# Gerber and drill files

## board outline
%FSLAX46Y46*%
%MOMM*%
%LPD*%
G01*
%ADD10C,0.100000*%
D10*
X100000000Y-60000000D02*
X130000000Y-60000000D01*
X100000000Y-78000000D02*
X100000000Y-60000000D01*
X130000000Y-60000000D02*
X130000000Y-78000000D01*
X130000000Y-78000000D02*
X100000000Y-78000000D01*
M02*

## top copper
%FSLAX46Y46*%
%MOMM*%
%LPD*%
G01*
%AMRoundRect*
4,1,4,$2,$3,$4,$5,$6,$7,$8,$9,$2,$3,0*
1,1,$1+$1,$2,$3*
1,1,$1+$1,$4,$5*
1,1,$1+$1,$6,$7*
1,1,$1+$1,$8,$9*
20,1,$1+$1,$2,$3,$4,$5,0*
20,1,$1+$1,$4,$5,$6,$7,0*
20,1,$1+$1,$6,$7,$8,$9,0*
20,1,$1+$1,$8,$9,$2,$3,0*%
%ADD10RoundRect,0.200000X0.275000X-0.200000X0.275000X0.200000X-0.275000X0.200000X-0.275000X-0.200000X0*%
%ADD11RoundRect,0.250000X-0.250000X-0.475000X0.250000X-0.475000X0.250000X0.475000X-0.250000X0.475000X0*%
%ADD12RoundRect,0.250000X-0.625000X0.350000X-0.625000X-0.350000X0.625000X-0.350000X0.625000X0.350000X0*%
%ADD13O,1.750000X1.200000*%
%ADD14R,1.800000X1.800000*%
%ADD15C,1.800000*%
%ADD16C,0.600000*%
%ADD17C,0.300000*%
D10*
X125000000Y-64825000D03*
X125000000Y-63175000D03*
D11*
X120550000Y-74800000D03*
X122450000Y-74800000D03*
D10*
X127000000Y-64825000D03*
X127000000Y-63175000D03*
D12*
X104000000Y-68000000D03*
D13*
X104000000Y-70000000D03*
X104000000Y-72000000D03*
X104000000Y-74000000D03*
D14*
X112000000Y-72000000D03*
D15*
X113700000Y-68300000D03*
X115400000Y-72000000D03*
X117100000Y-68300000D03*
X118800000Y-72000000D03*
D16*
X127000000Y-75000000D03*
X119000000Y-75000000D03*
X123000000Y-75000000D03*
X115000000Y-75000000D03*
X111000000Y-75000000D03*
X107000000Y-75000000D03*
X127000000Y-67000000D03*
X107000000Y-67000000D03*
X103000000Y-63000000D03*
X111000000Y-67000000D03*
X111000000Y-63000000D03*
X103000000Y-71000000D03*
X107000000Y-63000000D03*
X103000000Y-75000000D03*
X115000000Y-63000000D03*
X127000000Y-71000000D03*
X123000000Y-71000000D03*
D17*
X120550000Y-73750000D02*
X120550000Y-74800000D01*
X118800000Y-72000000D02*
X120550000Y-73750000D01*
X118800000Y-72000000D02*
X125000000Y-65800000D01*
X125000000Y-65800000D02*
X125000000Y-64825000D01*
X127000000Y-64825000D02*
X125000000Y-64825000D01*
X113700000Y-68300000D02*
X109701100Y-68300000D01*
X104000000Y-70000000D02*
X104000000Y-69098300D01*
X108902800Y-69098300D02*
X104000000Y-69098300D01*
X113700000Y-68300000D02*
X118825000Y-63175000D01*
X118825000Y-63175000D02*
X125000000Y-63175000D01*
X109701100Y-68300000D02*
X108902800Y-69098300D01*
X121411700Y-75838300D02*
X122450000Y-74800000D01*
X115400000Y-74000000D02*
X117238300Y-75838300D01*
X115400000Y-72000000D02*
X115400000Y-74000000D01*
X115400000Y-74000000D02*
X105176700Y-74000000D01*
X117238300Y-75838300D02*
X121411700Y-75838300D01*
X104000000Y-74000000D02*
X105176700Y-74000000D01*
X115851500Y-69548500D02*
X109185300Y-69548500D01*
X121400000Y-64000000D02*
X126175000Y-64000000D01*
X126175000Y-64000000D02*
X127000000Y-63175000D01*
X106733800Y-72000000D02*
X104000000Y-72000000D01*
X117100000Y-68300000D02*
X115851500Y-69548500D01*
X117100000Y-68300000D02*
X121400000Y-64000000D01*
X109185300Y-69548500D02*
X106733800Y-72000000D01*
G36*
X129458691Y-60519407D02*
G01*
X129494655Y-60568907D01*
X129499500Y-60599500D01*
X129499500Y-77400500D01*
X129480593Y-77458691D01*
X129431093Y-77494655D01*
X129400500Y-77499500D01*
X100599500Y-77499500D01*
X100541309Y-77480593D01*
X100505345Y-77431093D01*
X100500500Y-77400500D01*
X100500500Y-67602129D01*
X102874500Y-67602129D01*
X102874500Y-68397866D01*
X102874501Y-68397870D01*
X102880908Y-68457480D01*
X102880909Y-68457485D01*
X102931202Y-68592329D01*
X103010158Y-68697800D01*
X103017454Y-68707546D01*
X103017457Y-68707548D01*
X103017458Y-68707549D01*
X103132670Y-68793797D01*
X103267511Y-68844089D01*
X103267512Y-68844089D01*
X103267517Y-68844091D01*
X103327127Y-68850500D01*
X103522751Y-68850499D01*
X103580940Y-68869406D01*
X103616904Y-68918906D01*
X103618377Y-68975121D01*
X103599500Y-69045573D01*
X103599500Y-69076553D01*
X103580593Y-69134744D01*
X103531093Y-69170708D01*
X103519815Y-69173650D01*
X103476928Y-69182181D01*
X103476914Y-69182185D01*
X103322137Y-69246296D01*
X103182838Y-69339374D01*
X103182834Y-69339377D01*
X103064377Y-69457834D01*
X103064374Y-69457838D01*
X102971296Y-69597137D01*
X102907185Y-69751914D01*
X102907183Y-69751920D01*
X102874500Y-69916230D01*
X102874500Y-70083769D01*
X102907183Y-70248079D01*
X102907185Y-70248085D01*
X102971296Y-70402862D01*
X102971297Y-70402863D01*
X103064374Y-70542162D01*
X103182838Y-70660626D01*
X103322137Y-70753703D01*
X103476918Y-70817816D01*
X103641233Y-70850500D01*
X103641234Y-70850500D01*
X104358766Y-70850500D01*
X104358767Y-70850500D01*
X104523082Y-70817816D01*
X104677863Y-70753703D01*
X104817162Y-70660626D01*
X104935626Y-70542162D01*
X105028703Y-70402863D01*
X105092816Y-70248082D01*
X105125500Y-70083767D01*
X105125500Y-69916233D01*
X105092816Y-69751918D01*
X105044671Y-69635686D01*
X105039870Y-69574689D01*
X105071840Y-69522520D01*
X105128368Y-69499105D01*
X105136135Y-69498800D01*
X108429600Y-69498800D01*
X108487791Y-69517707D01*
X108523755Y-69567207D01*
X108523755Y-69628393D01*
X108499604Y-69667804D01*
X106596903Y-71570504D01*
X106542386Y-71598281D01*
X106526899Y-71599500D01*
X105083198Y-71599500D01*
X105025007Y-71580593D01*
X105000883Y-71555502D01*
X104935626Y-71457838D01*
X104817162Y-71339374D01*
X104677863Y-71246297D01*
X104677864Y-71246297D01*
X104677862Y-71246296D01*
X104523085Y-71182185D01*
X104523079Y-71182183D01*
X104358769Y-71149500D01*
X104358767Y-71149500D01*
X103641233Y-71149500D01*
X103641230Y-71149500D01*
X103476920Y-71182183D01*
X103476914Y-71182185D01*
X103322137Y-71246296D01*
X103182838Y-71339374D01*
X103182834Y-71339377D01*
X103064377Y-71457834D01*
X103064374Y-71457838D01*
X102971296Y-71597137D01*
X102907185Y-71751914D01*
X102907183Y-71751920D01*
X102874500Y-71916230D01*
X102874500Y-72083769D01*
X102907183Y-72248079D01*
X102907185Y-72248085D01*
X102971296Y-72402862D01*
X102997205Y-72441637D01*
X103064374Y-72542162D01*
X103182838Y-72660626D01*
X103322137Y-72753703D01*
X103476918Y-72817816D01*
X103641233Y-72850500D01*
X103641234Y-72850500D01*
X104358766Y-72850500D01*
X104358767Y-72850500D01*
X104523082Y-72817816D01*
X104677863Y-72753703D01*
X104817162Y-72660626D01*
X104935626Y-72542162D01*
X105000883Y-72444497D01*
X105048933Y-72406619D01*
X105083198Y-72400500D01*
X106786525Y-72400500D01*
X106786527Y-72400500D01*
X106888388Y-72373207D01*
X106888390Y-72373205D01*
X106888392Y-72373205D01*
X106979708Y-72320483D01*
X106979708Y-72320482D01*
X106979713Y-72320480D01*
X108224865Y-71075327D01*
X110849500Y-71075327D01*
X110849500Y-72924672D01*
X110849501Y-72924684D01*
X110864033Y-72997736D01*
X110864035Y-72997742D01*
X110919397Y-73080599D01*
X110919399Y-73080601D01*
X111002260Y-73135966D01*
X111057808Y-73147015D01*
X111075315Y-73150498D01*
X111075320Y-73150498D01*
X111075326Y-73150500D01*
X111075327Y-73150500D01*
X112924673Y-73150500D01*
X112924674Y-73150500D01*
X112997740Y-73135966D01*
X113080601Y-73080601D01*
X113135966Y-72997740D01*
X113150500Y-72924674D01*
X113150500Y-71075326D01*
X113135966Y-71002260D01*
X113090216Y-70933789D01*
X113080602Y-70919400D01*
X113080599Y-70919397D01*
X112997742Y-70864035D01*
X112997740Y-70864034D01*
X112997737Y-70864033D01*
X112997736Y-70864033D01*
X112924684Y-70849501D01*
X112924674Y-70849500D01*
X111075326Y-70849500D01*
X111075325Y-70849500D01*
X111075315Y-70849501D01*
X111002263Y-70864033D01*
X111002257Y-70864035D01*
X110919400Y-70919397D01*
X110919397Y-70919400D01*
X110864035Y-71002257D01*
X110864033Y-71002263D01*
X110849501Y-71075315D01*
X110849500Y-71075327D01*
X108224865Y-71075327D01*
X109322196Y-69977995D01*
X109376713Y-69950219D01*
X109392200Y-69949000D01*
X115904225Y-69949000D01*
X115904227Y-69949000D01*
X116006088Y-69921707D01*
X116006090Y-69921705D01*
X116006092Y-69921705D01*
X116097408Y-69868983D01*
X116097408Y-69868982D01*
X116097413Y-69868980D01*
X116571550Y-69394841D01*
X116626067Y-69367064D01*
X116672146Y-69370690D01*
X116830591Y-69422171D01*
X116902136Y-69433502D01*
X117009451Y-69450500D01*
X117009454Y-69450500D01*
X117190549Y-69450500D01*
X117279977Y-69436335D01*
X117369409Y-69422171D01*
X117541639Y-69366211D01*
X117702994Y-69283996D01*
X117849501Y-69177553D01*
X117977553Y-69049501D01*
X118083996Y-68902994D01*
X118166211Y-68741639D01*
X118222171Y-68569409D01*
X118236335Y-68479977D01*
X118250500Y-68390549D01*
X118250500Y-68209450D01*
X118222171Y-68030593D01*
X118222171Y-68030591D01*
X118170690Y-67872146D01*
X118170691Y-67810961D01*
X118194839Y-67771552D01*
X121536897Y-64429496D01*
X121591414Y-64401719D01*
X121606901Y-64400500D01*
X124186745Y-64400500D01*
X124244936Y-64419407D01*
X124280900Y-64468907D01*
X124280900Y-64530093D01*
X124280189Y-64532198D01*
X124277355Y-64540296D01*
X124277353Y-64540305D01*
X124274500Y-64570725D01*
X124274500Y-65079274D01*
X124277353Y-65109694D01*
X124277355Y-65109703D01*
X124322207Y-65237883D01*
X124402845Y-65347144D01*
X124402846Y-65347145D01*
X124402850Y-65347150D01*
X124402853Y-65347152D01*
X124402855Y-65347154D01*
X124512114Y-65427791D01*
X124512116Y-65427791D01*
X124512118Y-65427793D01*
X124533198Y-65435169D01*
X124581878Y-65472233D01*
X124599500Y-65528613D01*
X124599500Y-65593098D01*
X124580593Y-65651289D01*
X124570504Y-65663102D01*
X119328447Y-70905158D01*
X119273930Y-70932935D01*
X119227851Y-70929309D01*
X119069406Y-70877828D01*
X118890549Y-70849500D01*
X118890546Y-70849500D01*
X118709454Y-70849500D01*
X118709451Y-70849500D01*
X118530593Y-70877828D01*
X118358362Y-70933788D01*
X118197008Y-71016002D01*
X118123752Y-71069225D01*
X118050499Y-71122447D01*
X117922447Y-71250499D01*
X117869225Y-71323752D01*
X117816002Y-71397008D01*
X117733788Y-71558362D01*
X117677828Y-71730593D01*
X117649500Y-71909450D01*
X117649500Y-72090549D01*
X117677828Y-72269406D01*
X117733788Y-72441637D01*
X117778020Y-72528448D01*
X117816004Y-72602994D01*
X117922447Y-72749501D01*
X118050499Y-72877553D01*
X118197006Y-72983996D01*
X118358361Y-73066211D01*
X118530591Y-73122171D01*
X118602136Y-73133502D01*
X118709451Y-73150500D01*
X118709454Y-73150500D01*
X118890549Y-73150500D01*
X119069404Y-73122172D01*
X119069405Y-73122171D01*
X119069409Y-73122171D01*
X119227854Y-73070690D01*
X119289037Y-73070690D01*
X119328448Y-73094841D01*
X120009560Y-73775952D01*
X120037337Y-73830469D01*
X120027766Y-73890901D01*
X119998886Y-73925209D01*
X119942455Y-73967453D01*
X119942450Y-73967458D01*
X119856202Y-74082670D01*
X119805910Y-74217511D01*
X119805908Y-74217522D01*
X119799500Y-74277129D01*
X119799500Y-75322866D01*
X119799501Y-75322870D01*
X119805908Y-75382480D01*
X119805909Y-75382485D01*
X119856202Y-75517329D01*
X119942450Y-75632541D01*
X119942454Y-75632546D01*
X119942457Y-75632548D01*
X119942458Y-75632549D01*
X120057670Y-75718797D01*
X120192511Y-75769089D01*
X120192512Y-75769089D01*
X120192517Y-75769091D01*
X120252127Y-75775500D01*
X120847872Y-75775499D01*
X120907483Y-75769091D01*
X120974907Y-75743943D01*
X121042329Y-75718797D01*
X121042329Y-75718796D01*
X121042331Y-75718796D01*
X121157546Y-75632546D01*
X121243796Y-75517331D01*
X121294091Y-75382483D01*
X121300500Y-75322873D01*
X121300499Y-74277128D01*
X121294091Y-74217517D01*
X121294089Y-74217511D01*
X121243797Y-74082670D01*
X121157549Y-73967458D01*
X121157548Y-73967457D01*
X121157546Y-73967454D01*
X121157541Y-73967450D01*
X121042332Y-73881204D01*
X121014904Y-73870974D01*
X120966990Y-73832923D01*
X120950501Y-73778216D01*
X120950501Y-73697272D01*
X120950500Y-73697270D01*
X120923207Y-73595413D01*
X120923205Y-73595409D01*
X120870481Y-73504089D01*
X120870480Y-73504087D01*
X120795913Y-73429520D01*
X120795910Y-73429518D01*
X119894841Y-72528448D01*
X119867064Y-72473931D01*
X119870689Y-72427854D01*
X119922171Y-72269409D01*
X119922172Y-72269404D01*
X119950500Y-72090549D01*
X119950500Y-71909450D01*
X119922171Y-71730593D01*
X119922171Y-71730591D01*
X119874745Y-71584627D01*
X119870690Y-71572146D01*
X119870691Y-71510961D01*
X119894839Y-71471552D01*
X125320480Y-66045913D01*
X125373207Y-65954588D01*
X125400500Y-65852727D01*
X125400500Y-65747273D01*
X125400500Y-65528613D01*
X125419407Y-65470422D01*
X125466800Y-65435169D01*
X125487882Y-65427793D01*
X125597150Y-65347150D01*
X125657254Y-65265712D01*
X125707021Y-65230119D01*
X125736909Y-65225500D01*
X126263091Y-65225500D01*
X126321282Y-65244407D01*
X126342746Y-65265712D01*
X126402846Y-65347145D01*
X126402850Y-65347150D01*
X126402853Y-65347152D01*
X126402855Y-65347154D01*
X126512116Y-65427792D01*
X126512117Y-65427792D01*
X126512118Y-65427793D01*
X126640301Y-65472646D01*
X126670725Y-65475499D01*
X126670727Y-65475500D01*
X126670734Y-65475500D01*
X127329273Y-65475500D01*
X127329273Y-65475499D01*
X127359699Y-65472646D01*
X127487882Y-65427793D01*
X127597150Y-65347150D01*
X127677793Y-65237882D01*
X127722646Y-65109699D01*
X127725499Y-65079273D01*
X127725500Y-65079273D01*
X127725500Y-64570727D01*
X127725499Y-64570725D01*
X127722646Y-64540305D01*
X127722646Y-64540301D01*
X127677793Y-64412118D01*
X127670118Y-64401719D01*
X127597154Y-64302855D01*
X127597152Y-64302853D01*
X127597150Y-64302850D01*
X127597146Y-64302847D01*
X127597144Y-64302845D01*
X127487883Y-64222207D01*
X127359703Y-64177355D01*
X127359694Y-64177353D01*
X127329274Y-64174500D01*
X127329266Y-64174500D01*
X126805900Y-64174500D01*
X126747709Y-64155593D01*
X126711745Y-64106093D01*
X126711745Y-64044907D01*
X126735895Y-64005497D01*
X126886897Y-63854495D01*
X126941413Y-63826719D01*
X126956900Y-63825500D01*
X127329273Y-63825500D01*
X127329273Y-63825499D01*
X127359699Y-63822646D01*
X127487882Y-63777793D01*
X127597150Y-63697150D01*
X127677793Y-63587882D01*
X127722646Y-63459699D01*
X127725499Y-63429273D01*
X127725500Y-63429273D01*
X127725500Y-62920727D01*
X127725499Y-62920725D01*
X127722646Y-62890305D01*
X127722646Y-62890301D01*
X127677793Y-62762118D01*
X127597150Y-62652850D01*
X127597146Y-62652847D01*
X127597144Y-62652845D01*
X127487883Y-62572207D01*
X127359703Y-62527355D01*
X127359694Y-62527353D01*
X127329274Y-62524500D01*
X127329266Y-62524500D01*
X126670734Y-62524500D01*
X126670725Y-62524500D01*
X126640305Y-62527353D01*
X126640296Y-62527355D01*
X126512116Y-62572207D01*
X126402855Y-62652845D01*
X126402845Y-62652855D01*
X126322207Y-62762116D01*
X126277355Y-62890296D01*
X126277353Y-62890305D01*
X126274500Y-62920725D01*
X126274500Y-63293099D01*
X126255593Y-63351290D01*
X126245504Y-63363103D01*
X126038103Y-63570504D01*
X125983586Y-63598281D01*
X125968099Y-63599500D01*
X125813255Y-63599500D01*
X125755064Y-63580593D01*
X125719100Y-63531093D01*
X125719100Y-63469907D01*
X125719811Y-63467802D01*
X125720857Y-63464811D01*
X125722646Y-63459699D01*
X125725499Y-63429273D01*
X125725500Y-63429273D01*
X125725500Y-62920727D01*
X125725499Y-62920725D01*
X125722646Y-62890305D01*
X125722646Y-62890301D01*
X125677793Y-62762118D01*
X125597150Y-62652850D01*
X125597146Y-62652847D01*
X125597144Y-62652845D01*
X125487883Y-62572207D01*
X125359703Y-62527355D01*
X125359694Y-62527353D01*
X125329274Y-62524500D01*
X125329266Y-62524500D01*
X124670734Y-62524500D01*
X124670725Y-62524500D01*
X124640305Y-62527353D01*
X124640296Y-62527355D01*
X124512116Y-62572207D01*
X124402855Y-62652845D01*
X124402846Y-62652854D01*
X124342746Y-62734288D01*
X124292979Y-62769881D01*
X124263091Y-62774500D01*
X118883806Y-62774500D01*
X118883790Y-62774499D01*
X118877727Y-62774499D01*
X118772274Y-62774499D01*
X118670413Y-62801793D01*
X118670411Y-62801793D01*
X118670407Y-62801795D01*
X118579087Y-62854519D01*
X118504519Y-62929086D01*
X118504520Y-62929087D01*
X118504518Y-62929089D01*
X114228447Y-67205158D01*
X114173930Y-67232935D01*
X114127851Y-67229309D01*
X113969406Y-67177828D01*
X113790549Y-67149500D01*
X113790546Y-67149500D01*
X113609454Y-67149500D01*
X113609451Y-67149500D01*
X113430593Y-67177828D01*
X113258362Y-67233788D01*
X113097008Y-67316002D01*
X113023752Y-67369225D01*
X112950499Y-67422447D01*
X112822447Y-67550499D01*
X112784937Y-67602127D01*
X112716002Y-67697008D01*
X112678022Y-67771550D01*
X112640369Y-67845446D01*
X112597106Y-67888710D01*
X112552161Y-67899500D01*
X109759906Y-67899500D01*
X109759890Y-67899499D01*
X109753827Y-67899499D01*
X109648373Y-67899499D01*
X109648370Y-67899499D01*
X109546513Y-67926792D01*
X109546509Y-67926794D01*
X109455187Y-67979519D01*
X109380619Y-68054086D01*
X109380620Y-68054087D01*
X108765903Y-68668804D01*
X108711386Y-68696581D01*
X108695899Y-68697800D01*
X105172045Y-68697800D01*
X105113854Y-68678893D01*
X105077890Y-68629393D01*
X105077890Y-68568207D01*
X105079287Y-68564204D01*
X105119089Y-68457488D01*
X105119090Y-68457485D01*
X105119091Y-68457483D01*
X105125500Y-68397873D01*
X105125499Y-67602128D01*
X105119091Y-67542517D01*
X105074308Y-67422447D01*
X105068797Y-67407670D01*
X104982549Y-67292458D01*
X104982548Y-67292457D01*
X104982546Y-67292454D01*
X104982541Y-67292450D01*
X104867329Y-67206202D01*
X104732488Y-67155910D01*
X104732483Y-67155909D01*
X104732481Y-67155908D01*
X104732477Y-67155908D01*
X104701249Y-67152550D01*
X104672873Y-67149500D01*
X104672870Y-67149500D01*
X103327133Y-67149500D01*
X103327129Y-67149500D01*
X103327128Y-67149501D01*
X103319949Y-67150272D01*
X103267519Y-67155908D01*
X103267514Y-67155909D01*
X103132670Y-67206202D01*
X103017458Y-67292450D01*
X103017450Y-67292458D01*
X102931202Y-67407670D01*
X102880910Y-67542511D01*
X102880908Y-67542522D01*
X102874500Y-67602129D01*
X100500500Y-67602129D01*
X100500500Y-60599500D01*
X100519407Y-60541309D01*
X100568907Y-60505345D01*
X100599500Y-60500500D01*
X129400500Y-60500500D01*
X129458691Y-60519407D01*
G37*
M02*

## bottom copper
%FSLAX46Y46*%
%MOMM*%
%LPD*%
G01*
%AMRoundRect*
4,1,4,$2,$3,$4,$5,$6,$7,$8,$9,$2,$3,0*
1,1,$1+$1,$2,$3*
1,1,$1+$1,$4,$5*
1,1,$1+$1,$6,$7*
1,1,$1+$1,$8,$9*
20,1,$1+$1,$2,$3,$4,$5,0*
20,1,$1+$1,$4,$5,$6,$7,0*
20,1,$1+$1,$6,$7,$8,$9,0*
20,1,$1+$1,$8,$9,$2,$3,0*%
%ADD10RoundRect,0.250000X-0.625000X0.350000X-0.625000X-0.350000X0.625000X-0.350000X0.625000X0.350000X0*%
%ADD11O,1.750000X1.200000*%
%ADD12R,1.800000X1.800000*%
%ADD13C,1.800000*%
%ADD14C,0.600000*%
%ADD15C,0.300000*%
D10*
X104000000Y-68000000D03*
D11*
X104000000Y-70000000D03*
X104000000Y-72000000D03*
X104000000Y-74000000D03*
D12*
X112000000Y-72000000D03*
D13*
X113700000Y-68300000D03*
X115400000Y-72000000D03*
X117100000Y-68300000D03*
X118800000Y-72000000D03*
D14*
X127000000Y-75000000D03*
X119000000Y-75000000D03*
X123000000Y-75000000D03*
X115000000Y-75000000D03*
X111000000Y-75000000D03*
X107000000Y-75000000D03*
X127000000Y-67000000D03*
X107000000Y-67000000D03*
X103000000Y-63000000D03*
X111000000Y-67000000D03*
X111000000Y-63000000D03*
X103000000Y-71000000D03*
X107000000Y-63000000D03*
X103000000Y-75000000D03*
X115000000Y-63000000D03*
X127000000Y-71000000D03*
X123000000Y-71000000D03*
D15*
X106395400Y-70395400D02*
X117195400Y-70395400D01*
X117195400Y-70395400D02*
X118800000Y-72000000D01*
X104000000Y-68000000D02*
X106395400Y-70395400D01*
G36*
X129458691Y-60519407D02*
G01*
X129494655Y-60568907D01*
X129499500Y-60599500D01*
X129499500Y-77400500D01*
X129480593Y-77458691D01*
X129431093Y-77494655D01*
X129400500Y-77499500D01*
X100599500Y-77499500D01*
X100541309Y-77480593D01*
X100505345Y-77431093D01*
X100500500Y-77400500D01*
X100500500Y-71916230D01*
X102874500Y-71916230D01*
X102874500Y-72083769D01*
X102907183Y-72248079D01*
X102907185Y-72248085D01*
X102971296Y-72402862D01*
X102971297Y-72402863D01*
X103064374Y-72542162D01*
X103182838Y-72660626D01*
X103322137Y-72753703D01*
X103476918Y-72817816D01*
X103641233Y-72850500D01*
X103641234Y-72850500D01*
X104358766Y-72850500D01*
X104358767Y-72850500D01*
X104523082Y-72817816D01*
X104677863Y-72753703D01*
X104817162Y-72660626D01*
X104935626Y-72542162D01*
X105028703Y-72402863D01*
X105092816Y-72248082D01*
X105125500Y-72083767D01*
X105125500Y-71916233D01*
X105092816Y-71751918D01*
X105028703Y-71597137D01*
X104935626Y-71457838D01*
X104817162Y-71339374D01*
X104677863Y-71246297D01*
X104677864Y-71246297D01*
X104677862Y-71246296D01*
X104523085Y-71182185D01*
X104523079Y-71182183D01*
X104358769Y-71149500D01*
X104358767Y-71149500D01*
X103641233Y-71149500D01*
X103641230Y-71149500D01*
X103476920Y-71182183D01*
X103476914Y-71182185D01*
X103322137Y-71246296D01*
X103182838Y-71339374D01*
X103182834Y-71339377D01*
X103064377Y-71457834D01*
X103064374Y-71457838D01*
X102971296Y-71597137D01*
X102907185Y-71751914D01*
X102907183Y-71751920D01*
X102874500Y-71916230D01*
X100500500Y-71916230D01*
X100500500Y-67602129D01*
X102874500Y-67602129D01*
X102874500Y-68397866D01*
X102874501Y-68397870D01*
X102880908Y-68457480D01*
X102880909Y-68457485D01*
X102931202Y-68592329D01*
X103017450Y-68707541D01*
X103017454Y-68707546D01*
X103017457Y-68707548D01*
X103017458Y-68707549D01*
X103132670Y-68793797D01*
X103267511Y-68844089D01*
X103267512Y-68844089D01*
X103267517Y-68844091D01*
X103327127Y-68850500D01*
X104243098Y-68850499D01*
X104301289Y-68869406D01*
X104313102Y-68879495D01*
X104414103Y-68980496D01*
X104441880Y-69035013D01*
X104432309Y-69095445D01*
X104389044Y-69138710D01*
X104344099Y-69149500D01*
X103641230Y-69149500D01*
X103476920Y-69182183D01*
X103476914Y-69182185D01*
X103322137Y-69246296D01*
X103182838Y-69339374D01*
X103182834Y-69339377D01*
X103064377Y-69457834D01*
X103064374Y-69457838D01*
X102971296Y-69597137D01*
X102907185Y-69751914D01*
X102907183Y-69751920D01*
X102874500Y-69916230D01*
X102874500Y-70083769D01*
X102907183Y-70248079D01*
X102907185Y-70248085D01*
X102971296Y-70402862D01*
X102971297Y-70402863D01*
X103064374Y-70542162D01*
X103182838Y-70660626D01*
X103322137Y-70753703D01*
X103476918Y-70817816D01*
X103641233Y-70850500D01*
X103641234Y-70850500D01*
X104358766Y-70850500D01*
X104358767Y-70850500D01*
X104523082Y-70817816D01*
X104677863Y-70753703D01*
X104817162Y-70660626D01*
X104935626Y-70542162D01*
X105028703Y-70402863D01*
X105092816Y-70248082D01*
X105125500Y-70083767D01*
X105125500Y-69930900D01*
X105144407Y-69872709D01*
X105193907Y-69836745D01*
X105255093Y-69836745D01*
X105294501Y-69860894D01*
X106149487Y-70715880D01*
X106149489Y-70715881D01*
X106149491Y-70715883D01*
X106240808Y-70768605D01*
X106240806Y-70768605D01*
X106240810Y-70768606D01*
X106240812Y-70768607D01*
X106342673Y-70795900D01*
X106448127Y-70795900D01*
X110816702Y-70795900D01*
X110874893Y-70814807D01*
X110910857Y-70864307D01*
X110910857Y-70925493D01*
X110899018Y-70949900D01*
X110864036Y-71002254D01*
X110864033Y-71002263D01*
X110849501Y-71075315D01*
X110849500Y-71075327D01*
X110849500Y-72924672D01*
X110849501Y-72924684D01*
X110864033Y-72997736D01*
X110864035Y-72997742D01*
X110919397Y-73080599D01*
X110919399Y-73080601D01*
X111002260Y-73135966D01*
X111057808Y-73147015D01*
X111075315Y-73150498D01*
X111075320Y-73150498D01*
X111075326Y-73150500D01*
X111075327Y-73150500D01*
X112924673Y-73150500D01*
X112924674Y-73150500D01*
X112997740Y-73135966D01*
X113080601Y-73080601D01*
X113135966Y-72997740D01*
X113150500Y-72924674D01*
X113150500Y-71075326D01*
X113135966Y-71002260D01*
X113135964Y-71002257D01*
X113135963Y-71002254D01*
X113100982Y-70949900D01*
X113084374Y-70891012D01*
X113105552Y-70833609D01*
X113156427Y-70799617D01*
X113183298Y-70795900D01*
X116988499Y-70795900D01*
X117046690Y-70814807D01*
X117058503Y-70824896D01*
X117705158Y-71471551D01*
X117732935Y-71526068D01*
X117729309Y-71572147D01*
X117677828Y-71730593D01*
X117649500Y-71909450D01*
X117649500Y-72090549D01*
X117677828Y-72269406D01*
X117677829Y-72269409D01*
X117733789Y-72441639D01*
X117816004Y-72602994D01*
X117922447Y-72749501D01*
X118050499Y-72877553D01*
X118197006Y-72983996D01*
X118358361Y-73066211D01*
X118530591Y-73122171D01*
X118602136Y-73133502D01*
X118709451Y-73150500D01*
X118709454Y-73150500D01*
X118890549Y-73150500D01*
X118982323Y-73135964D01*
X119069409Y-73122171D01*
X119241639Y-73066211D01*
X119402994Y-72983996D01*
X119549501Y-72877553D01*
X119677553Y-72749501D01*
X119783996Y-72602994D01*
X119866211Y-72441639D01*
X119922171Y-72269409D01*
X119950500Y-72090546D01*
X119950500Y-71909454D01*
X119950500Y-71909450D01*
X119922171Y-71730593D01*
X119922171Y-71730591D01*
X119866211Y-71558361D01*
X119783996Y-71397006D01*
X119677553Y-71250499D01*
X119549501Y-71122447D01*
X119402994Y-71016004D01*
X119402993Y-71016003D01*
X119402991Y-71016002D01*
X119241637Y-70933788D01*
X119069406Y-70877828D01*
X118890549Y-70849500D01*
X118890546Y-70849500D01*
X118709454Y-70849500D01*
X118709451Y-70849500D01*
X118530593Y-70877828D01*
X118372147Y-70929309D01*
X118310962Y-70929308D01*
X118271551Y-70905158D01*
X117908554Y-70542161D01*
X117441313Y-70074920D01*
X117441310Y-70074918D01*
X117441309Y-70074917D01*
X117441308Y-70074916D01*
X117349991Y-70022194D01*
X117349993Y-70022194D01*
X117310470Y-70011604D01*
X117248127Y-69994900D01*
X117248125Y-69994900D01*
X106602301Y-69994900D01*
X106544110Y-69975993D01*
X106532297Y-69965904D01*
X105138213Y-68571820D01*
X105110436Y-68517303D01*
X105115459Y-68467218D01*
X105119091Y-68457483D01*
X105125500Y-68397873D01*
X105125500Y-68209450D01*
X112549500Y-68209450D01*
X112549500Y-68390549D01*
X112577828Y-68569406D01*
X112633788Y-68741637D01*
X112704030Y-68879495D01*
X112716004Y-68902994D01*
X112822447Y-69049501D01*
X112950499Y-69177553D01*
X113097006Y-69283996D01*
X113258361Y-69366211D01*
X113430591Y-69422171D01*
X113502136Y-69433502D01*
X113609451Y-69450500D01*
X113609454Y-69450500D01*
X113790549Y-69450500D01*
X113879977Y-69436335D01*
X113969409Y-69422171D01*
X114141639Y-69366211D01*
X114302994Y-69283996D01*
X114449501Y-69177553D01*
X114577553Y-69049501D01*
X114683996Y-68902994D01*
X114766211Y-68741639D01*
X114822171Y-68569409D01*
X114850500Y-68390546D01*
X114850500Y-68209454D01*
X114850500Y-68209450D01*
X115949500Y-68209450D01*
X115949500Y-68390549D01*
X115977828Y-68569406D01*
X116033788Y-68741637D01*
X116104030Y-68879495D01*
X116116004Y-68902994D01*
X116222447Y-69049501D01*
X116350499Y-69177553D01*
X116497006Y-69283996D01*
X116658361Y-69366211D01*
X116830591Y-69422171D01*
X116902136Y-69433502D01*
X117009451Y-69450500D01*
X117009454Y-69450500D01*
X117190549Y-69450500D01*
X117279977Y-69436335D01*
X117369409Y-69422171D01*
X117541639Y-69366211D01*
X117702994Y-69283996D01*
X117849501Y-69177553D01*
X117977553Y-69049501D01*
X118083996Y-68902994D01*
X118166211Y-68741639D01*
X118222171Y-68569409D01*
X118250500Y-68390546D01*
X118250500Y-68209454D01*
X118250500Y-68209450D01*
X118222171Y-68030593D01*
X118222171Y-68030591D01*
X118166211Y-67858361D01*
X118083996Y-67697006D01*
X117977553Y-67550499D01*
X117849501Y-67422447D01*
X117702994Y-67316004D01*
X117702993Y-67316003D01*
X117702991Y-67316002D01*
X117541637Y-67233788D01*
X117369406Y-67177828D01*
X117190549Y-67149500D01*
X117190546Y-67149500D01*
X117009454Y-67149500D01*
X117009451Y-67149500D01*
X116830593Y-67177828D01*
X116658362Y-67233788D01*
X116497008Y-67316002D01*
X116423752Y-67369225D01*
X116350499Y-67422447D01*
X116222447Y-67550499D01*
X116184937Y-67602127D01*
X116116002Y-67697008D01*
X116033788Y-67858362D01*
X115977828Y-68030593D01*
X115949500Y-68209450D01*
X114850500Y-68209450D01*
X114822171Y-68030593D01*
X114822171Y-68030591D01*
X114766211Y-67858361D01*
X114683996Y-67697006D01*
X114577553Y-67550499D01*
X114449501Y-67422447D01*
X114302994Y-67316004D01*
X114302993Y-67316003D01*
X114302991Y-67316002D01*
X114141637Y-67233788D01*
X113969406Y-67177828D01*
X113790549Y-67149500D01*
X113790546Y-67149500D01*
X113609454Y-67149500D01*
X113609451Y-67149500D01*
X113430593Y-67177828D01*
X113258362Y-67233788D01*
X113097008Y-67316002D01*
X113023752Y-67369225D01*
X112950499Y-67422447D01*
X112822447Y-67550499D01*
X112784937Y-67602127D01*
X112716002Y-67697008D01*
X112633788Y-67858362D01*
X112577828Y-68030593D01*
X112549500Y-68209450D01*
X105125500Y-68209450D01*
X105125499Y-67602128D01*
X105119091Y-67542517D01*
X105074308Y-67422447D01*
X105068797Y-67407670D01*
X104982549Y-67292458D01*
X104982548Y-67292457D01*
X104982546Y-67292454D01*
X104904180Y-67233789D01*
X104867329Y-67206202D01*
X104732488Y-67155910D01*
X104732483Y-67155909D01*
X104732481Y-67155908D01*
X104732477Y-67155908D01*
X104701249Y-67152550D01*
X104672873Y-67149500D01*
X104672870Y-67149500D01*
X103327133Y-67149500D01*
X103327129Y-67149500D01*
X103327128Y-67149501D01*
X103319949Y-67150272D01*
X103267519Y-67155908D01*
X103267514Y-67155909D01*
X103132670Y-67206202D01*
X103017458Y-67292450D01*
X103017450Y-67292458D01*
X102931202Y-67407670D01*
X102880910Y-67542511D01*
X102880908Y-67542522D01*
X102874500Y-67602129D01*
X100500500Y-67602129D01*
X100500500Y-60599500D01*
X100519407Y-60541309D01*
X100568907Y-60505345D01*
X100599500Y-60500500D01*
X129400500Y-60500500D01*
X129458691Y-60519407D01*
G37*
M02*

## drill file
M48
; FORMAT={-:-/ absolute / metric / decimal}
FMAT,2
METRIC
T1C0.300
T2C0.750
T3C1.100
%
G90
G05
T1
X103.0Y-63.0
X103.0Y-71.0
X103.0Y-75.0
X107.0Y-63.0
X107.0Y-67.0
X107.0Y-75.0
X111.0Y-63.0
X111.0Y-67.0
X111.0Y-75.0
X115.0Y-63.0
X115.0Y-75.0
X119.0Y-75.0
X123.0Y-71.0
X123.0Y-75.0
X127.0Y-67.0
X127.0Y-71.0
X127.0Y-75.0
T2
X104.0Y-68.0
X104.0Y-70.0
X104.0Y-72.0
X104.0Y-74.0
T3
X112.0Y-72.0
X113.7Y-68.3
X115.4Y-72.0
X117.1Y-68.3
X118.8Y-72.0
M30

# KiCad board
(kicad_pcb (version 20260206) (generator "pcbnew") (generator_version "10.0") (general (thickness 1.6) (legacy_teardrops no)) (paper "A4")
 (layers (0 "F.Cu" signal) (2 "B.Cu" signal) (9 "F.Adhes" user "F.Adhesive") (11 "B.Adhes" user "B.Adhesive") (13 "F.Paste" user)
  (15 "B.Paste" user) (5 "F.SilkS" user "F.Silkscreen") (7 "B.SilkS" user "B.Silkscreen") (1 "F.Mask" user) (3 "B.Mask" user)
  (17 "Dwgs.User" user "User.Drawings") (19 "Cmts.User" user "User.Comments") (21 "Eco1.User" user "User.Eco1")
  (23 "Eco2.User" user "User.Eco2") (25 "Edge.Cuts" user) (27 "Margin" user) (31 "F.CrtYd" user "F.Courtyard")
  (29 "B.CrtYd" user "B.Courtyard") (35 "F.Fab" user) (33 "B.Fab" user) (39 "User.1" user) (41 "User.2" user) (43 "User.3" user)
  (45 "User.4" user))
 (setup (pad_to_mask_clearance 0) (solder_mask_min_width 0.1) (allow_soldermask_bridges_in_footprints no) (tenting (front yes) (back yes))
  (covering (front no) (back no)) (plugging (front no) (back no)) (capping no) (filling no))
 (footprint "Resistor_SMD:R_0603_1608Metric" (layer "F.Cu") (at 125 64 90)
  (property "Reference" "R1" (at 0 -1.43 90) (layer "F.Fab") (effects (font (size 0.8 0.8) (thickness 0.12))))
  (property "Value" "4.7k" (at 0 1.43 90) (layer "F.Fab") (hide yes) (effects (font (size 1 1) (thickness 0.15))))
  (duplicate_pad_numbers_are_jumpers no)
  (pad "1" smd roundrect (at -0.825 0 90) (size 0.8 0.95) (layers "F.Cu" "F.Mask" "F.Paste") (roundrect_rratio 0.25) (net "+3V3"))
  (pad "2" smd roundrect (at 0.825 0 90) (size 0.8 0.95) (layers "F.Cu" "F.Mask" "F.Paste") (roundrect_rratio 0.25) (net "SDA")))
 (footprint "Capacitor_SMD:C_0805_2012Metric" (layer "F.Cu") (at 121.5 74.8)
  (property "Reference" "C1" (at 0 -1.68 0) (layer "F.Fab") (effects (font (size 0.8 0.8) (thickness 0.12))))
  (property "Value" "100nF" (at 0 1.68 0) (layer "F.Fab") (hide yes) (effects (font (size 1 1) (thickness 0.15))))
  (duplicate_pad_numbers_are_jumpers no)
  (pad "1" smd roundrect (at -0.95 0) (size 1 1.45) (layers "F.Cu" "F.Mask" "F.Paste") (roundrect_rratio 0.25) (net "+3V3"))
  (pad "2" smd roundrect (at 0.95 0) (size 1 1.45) (layers "F.Cu" "F.Mask" "F.Paste") (roundrect_rratio 0.25) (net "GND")))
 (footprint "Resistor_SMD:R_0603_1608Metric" (layer "F.Cu") (at 127 64 90)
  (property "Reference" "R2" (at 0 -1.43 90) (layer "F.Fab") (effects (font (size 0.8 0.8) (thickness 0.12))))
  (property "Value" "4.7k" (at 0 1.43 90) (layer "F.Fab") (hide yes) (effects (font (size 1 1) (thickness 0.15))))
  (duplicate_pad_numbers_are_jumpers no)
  (pad "1" smd roundrect (at -0.825 0 90) (size 0.8 0.95) (layers "F.Cu" "F.Mask" "F.Paste") (roundrect_rratio 0.25) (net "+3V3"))
  (pad "2" smd roundrect (at 0.825 0 90) (size 0.8 0.95) (layers "F.Cu" "F.Mask" "F.Paste") (roundrect_rratio 0.25) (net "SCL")))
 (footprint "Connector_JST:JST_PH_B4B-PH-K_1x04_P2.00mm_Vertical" (layer "F.Cu") (at 104 68 -90)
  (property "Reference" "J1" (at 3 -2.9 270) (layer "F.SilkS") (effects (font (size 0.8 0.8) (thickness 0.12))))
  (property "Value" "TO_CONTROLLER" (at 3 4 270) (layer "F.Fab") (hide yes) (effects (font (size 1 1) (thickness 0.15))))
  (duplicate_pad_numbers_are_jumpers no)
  (pad "1" thru_hole roundrect (at 0 0 270) (size 1.2 1.75) (drill 0.75) (layers "*.Cu" "*.Mask") (remove_unused_layers no)
   (roundrect_rratio 0.208333) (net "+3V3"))
  (pad "2" thru_hole oval (at 2 0 270) (size 1.2 1.75) (drill 0.75) (layers "*.Cu" "*.Mask") (remove_unused_layers no) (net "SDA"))
  (pad "3" thru_hole oval (at 4 0 270) (size 1.2 1.75) (drill 0.75) (layers "*.Cu" "*.Mask") (remove_unused_layers no) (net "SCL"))
  (pad "4" thru_hole oval (at 6 0 270) (size 1.2 1.75) (drill 0.75) (layers "*.Cu" "*.Mask") (remove_unused_layers no) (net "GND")))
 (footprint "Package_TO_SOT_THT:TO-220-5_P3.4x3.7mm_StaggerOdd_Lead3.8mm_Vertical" (layer "F.Cu") (at 112 72)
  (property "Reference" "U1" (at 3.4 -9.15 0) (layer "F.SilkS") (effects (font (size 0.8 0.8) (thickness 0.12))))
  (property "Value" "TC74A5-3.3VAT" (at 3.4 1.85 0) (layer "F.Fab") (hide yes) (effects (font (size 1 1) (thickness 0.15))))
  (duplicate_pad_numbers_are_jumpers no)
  (pad "1" thru_hole rect (at 0 0) (size 1.8 1.8) (drill 1.1) (layers "*.Cu" "*.Mask") (remove_unused_layers no))
  (pad "2" thru_hole circle (at 1.7 -3.7) (size 1.8 1.8) (drill 1.1) (layers "*.Cu" "*.Mask") (remove_unused_layers no) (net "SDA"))
  (pad "3" thru_hole circle (at 3.4 0) (size 1.8 1.8) (drill 1.1) (layers "*.Cu" "*.Mask") (remove_unused_layers no) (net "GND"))
  (pad "4" thru_hole circle (at 5.1 -3.7) (size 1.8 1.8) (drill 1.1) (layers "*.Cu" "*.Mask") (remove_unused_layers no) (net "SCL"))
  (pad "5" thru_hole circle (at 6.8 0) (size 1.8 1.8) (drill 1.1) (layers "*.Cu" "*.Mask") (remove_unused_layers no) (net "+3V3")))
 (gr_line (start 100 60) (end 130 60) (stroke (width 0.1) (type default)) (layer "Edge.Cuts"))
 (gr_line (start 100 78) (end 100 60) (stroke (width 0.1) (type default)) (layer "Edge.Cuts"))
 (gr_line (start 130 60) (end 130 78) (stroke (width 0.1) (type default)) (layer "Edge.Cuts"))
 (gr_line (start 130 78) (end 100 78) (stroke (width 0.1) (type default)) (layer "Edge.Cuts"))
 (segment (start 120.55 73.75) (end 120.55 74.8) (width 0.3) (layer "F.Cu") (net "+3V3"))
 (segment (start 118.8 72) (end 120.55 73.75) (width 0.3) (layer "F.Cu") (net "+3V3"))
 (segment (start 118.8 72) (end 125 65.8) (width 0.3) (layer "F.Cu") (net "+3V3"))
 (segment (start 125 65.8) (end 125 64.825) (width 0.3) (layer "F.Cu") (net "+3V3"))
 (segment (start 127 64.825) (end 125 64.825) (width 0.3) (layer "F.Cu") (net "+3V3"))
 (segment (start 106.3954 70.3954) (end 117.1954 70.3954) (width 0.3) (layer "B.Cu") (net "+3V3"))
 (segment (start 117.1954 70.3954) (end 118.8 72) (width 0.3) (layer "B.Cu") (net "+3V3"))
 (segment (start 104 68) (end 106.3954 70.3954) (width 0.3) (layer "B.Cu") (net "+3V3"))
 (segment (start 113.7 68.3) (end 109.7011 68.3) (width 0.3) (layer "F.Cu") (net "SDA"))
 (segment (start 104 70) (end 104 69.0983) (width 0.3) (layer "F.Cu") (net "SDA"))
 (segment (start 108.9028 69.0983) (end 104 69.0983) (width 0.3) (layer "F.Cu") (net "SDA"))
 (segment (start 113.7 68.3) (end 118.825 63.175) (width 0.3) (layer "F.Cu") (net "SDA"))
 (segment (start 118.825 63.175) (end 125 63.175) (width 0.3) (layer "F.Cu") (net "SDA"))
 (segment (start 109.7011 68.3) (end 108.9028 69.0983) (width 0.3) (layer "F.Cu") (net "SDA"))
 (segment (start 121.4117 75.8383) (end 122.45 74.8) (width 0.3) (layer "F.Cu") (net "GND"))
 (segment (start 115.4 74) (end 117.2383 75.8383) (width 0.3) (layer "F.Cu") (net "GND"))
 (segment (start 115.4 72) (end 115.4 74) (width 0.3) (layer "F.Cu") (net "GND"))
 (segment (start 115.4 74) (end 105.1767 74) (width 0.3) (layer "F.Cu") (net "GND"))
 (segment (start 117.2383 75.8383) (end 121.4117 75.8383) (width 0.3) (layer "F.Cu") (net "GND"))
 (segment (start 104 74) (end 105.1767 74) (width 0.3) (layer "F.Cu") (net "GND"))
 (via (at 127 75) (size 0.6) (drill 0.3) (layers "F.Cu" "B.Cu") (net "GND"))
 (via (at 119 75) (size 0.6) (drill 0.3) (layers "F.Cu" "B.Cu") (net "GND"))
 (via (at 123 75) (size 0.6) (drill 0.3) (layers "F.Cu" "B.Cu") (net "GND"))
 (via (at 115 75) (size 0.6) (drill 0.3) (layers "F.Cu" "B.Cu") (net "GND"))
 (via (at 111 75) (size 0.6) (drill 0.3) (layers "F.Cu" "B.Cu") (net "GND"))
 (via (at 107 75) (size 0.6) (drill 0.3) (layers "F.Cu" "B.Cu") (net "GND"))
 (via (at 127 67) (size 0.6) (drill 0.3) (layers "F.Cu" "B.Cu") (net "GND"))
 (via (at 107 67) (size 0.6) (drill 0.3) (layers "F.Cu" "B.Cu") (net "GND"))
 (via (at 103 63) (size 0.6) (drill 0.3) (layers "F.Cu" "B.Cu") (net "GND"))
 (via (at 111 67) (size 0.6) (drill 0.3) (layers "F.Cu" "B.Cu") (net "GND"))
 (via (at 111 63) (size 0.6) (drill 0.3) (layers "F.Cu" "B.Cu") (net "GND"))
 (via (at 103 71) (size 0.6) (drill 0.3) (layers "F.Cu" "B.Cu") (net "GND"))
 (via (at 107 63) (size 0.6) (drill 0.3) (layers "F.Cu" "B.Cu") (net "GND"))
 (via (at 103 75) (size 0.6) (drill 0.3) (layers "F.Cu" "B.Cu") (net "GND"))
 (via (at 115 63) (size 0.6) (drill 0.3) (layers "F.Cu" "B.Cu") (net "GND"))
 (via (at 127 71) (size 0.6) (drill 0.3) (layers "F.Cu" "B.Cu") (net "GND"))
 (via (at 123 71) (size 0.6) (drill 0.3) (layers "F.Cu" "B.Cu") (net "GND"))
 (segment (start 115.8515 69.5485) (end 109.1853 69.5485) (width 0.3) (layer "F.Cu") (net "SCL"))
 (segment (start 121.4 64) (end 126.175 64) (width 0.3) (layer "F.Cu") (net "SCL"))
 (segment (start 126.175 64) (end 127 63.175) (width 0.3) (layer "F.Cu") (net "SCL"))
 (segment (start 106.7338 72) (end 104 72) (width 0.3) (layer "F.Cu") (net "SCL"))
 (segment (start 117.1 68.3) (end 115.8515 69.5485) (width 0.3) (layer "F.Cu") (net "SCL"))
 (segment (start 117.1 68.3) (end 121.4 64) (width 0.3) (layer "F.Cu") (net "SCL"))
 (segment (start 109.1853 69.5485) (end 106.7338 72) (width 0.3) (layer "F.Cu") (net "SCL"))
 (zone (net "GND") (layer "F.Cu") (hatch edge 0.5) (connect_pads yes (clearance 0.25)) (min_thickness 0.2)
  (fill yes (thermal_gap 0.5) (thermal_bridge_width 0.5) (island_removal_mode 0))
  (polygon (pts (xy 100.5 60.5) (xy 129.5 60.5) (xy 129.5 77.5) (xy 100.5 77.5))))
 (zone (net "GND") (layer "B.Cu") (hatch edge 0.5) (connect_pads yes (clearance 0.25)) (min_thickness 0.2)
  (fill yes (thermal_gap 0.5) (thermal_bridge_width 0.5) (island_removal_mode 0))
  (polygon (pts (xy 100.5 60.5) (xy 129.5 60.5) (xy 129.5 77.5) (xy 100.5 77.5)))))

